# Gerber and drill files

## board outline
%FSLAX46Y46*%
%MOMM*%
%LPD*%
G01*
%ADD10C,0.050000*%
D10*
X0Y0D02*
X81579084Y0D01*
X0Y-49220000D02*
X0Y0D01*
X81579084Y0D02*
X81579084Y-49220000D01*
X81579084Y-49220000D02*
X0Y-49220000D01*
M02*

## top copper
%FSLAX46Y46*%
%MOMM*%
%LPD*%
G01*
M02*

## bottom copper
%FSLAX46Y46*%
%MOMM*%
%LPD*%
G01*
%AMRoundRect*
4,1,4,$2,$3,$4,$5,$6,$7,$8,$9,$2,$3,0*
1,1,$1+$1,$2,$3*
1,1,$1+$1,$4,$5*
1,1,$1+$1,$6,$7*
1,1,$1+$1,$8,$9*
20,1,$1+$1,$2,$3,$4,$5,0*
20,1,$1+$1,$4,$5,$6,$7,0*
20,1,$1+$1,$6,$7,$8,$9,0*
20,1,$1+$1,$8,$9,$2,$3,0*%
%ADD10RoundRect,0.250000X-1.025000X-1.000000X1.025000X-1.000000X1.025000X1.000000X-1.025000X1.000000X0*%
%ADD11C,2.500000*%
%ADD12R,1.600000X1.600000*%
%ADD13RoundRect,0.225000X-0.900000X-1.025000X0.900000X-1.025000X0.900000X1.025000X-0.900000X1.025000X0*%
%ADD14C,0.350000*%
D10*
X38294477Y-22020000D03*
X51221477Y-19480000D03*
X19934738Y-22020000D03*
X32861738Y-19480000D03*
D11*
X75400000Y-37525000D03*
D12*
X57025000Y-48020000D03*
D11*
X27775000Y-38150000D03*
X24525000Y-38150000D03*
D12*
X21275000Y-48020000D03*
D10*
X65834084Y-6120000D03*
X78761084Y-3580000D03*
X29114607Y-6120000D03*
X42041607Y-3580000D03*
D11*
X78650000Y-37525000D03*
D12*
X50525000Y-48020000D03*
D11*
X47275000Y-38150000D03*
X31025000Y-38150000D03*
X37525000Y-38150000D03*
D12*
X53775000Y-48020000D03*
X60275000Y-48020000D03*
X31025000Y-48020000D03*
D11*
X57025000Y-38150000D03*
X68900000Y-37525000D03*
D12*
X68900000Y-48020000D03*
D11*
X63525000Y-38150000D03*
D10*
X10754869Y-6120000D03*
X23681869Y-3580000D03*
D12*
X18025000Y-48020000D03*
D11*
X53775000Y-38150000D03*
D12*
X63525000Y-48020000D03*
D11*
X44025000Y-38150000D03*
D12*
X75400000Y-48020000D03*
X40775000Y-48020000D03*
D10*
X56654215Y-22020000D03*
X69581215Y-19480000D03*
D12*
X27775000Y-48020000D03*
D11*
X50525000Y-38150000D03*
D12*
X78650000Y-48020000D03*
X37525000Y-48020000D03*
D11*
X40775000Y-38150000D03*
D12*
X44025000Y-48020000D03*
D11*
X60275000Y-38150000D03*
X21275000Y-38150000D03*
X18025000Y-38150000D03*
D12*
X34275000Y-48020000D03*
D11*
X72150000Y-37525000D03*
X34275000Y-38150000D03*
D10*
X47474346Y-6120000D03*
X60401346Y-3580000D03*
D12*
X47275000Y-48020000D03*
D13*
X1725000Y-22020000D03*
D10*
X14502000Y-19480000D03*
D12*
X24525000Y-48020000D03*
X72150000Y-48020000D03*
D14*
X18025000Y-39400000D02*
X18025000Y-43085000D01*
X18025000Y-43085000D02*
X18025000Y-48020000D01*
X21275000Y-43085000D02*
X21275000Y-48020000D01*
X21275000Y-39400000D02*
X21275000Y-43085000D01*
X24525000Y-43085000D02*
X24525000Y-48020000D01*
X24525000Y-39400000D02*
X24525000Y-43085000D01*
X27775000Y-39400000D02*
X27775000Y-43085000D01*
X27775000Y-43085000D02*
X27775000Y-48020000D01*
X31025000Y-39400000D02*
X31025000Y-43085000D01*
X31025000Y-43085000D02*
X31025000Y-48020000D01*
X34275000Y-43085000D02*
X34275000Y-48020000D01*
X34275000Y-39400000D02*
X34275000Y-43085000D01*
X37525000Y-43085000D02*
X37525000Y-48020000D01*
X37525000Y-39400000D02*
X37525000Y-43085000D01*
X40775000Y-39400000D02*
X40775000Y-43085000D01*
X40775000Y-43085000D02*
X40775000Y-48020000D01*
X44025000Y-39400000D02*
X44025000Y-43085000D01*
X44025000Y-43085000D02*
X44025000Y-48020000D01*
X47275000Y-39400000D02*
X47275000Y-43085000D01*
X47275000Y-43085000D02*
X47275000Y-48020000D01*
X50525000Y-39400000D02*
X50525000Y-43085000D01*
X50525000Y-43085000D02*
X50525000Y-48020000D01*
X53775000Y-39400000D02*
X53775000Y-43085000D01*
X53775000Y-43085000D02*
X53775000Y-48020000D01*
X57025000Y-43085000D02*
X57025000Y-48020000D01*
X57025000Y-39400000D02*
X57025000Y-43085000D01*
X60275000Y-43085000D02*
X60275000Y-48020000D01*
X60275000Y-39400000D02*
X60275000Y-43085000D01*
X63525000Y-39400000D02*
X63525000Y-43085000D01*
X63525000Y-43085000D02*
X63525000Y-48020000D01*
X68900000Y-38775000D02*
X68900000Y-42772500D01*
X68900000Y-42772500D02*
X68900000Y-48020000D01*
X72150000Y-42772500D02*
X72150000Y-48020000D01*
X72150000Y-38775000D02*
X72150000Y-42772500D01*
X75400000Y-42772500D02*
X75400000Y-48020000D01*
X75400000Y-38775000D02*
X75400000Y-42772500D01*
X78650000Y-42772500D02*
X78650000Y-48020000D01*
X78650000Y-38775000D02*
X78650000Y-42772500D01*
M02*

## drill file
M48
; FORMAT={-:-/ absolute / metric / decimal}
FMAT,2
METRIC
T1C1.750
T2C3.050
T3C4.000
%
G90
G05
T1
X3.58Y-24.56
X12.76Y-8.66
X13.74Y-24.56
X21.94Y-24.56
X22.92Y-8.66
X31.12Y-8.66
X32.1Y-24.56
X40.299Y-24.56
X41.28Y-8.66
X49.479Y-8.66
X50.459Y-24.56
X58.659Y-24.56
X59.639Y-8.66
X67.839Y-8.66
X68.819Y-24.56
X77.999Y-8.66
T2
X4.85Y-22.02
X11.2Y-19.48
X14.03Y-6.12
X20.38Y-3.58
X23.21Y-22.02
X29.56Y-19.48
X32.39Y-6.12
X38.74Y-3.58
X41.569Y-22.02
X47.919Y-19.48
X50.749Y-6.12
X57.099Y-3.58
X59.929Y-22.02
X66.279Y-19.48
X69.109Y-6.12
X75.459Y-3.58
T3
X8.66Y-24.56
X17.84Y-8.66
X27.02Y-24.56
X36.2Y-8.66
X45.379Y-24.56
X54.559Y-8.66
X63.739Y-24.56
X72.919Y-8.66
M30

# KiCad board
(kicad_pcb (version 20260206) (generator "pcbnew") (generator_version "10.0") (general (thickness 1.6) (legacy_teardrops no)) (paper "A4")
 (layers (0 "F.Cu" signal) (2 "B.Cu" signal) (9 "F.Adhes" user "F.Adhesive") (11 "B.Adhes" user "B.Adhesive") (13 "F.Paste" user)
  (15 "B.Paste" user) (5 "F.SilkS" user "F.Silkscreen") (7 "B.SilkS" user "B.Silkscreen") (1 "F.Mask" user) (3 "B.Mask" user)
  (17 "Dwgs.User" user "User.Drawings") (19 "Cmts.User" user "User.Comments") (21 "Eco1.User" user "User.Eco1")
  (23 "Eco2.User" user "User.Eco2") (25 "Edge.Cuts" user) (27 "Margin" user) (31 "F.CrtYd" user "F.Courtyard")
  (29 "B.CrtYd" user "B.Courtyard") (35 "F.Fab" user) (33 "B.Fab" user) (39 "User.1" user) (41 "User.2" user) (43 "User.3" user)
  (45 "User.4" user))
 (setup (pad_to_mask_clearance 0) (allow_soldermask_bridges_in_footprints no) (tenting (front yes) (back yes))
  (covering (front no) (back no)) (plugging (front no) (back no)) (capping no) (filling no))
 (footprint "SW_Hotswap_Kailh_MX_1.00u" (layer "F.Cu") (at 45.379477 24.56)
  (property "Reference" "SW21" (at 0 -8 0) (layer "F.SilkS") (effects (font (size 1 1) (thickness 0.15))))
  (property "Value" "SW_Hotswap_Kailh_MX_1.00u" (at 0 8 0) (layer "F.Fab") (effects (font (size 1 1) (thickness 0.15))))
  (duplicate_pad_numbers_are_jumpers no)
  (pad "" np_thru_hole circle (at -5.08 0) (size 1.75 1.75) (drill 1.75) (layers "*.Cu" "*.Mask"))
  (pad "" np_thru_hole circle (at -3.81 -2.54) (size 3.05 3.05) (drill 3.05) (layers "*.Cu" "*.Mask"))
  (pad "" np_thru_hole circle (at 0 0) (size 4 4) (drill 4) (layers "*.Cu" "*.Mask"))
  (pad "" np_thru_hole circle (at 2.54 -5.08) (size 3.05 3.05) (drill 3.05) (layers "*.Cu" "*.Mask"))
  (pad "" np_thru_hole circle (at 5.08 0) (size 1.75 1.75) (drill 1.75) (layers "*.Cu" "*.Mask"))
  (pad "1" smd roundrect (at -7.085 -2.54) (size 2.55 2.5) (layers "B.Cu" "B.Mask" "B.Paste") (roundrect_rratio 0.1))
  (pad "2" smd roundrect (at 5.842 -5.08) (size 2.55 2.5) (layers "B.Cu" "B.Mask" "B.Paste") (roundrect_rratio 0.1)))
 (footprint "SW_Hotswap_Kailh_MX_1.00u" (layer "F.Cu") (at 27.019738 24.56)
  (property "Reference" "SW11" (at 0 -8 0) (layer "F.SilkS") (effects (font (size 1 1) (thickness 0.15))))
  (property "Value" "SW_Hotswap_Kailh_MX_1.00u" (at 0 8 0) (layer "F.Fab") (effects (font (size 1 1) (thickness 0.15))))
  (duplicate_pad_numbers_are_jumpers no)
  (pad "" np_thru_hole circle (at -5.08 0) (size 1.75 1.75) (drill 1.75) (layers "*.Cu" "*.Mask"))
  (pad "" np_thru_hole circle (at -3.81 -2.54) (size 3.05 3.05) (drill 3.05) (layers "*.Cu" "*.Mask"))
  (pad "" np_thru_hole circle (at 0 0) (size 4 4) (drill 4) (layers "*.Cu" "*.Mask"))
  (pad "" np_thru_hole circle (at 2.54 -5.08) (size 3.05 3.05) (drill 3.05) (layers "*.Cu" "*.Mask"))
  (pad "" np_thru_hole circle (at 5.08 0) (size 1.75 1.75) (drill 1.75) (layers "*.Cu" "*.Mask"))
  (pad "1" smd roundrect (at -7.085 -2.54) (size 2.55 2.5) (layers "B.Cu" "B.Mask" "B.Paste") (roundrect_rratio 0.1))
  (pad "2" smd roundrect (at 5.842 -5.08) (size 2.55 2.5) (layers "B.Cu" "B.Mask" "B.Paste") (roundrect_rratio 0.1)))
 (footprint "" (layer "F.Cu") (at 0 0)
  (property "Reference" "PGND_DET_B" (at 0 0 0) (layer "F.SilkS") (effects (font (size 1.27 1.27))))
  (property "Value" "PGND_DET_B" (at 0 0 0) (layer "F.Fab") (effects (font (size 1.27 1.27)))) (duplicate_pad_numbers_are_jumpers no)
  (pad "1" smd circle (at 75.4 37.525) (size 2.5 2.5) (layers "B.Cu" "B.Mask") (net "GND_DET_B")))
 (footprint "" (layer "F.Cu") (at 0 0)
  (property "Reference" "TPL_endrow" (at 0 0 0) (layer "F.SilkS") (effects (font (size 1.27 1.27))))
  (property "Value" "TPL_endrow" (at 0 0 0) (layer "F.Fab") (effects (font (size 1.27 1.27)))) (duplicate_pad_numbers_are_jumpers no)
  (pad "1" smd rect (at 57.025 48.02) (size 1.6 1.6) (layers "B.Cu" "B.Mask") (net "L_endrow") (thermal_bridge_angle 45)))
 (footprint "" (layer "F.Cu") (at 0 0)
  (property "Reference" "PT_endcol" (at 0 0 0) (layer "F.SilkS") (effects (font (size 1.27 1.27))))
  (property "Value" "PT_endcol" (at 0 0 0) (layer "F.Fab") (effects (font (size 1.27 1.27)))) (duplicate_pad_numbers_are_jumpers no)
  (pad "1" smd circle (at 27.775 38.15) (size 2.5 2.5) (layers "B.Cu" "B.Mask") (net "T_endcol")))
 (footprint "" (layer "F.Cu") (at 0 0)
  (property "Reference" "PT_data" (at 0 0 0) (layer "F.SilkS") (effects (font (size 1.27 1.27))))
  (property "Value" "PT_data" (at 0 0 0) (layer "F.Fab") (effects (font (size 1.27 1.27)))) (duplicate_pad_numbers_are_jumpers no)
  (pad "1" smd circle (at 24.525 38.15) (size 2.5 2.5) (layers "B.Cu" "B.Mask") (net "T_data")))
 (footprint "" (layer "F.Cu") (at 0 0)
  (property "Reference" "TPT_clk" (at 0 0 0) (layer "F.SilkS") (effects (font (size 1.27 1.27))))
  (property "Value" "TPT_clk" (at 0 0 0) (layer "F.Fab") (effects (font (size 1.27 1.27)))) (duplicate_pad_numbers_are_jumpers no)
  (pad "1" smd rect (at 21.275 48.02) (size 1.6 1.6) (layers "B.Cu" "B.Mask") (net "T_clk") (thermal_bridge_angle 45)))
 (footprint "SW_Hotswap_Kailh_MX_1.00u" (layer "F.Cu") (at 72.919084 8.66)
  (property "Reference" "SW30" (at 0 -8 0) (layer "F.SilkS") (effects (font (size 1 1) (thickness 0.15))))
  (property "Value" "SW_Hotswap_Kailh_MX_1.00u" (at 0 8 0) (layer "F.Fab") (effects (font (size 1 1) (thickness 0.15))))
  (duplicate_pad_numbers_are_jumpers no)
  (pad "" np_thru_hole circle (at -5.08 0) (size 1.75 1.75) (drill 1.75) (layers "*.Cu" "*.Mask"))
  (pad "" np_thru_hole circle (at -3.81 -2.54) (size 3.05 3.05) (drill 3.05) (layers "*.Cu" "*.Mask"))
  (pad "" np_thru_hole circle (at 0 0) (size 4 4) (drill 4) (layers "*.Cu" "*.Mask"))
  (pad "" np_thru_hole circle (at 2.54 -5.08) (size 3.05 3.05) (drill 3.05) (layers "*.Cu" "*.Mask"))
  (pad "" np_thru_hole circle (at 5.08 0) (size 1.75 1.75) (drill 1.75) (layers "*.Cu" "*.Mask"))
  (pad "1" smd roundrect (at -7.085 -2.54) (size 2.55 2.5) (layers "B.Cu" "B.Mask" "B.Paste") (roundrect_rratio 0.1))
  (pad "2" smd roundrect (at 5.842 -5.08) (size 2.55 2.5) (layers "B.Cu" "B.Mask" "B.Paste") (roundrect_rratio 0.1)))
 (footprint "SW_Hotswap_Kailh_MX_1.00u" (layer "F.Cu") (at 36.199607 8.66)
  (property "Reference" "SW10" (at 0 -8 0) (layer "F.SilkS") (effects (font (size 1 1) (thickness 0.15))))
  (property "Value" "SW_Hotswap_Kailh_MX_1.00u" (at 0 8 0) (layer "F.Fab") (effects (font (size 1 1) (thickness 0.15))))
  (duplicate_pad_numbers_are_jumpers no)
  (pad "" np_thru_hole circle (at -5.08 0) (size 1.75 1.75) (drill 1.75) (layers "*.Cu" "*.Mask"))
  (pad "" np_thru_hole circle (at -3.81 -2.54) (size 3.05 3.05) (drill 3.05) (layers "*.Cu" "*.Mask"))
  (pad "" np_thru_hole circle (at 0 0) (size 4 4) (drill 4) (layers "*.Cu" "*.Mask"))
  (pad "" np_thru_hole circle (at 2.54 -5.08) (size 3.05 3.05) (drill 3.05) (layers "*.Cu" "*.Mask"))
  (pad "" np_thru_hole circle (at 5.08 0) (size 1.75 1.75) (drill 1.75) (layers "*.Cu" "*.Mask"))
  (pad "1" smd roundrect (at -7.085 -2.54) (size 2.55 2.5) (layers "B.Cu" "B.Mask" "B.Paste") (roundrect_rratio 0.1))
  (pad "2" smd roundrect (at 5.842 -5.08) (size 2.55 2.5) (layers "B.Cu" "B.Mask" "B.Paste") (roundrect_rratio 0.1)))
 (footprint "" (layer "F.Cu") (at 0 0)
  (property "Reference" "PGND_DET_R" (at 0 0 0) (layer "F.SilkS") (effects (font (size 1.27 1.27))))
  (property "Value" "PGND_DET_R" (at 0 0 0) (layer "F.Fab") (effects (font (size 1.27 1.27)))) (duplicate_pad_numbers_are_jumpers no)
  (pad "1" smd circle (at 78.65 37.525) (size 2.5 2.5) (layers "B.Cu" "B.Mask") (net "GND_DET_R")))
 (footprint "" (layer "F.Cu") (at 0 0)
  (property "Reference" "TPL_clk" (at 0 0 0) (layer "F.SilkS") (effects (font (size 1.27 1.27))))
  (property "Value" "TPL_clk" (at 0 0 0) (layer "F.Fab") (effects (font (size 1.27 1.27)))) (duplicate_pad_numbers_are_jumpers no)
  (pad "1" smd rect (at 50.525 48.02) (size 1.6 1.6) (layers "B.Cu" "B.Mask") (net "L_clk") (thermal_bridge_angle 45)))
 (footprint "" (layer "F.Cu") (at 0 0)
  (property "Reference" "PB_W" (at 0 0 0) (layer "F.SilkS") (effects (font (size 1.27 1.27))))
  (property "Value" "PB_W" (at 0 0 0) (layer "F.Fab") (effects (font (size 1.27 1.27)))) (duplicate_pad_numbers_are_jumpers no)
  (pad "1" smd circle (at 47.275 38.15) (size 2.5 2.5) (layers "B.Cu" "B.Mask") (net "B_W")))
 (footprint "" (layer "F.Cu") (at 0 0)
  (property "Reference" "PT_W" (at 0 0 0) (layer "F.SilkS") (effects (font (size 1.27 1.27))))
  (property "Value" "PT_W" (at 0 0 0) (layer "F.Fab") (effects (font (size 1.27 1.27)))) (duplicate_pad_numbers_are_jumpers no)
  (pad "1" smd circle (at 31.025 38.15) (size 2.5 2.5) (layers "B.Cu" "B.Mask") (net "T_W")))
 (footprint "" (layer "F.Cu") (at 0 0)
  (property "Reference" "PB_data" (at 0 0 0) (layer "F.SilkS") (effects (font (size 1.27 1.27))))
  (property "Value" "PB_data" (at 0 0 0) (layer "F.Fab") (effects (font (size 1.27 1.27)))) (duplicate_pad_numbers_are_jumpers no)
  (pad "1" smd circle (at 37.525 38.15) (size 2.5 2.5) (layers "B.Cu" "B.Mask") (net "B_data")))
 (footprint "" (layer "F.Cu") (at 0 0)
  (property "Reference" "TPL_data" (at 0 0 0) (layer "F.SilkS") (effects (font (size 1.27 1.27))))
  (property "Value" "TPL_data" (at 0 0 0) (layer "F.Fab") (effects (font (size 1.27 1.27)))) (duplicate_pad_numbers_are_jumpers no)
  (pad "1" smd rect (at 53.775 48.02) (size 1.6 1.6) (layers "B.Cu" "B.Mask") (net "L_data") (thermal_bridge_angle 45)))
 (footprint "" (layer "F.Cu") (at 0 0)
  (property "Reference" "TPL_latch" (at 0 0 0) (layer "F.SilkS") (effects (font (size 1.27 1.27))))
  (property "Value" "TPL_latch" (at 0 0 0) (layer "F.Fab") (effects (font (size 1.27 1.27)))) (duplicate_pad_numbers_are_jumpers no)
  (pad "1" smd rect (at 60.275 48.02) (size 1.6 1.6) (layers "B.Cu" "B.Mask") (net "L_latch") (thermal_bridge_angle 45)))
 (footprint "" (layer "F.Cu") (at 0 0)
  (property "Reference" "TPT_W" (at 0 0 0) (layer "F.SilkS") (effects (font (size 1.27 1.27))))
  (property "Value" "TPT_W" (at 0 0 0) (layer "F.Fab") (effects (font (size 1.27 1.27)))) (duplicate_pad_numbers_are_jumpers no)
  (pad "1" smd rect (at 31.025 48.02) (size 1.6 1.6) (layers "B.Cu" "B.Mask") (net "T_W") (thermal_bridge_angle 45)))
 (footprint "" (layer "F.Cu") (at 0 0)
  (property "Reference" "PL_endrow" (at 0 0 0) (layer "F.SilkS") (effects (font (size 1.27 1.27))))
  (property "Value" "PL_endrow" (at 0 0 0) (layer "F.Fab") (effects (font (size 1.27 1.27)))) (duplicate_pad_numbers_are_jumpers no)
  (pad "1" smd circle (at 57.025 38.15) (size 2.5 2.5) (layers "B.Cu" "B.Mask") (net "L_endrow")))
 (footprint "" (layer "F.Cu") (at 0 0)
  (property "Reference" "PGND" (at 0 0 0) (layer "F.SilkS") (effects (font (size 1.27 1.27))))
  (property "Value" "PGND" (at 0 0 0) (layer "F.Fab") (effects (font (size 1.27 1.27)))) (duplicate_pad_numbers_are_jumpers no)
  (pad "1" smd circle (at 68.9 37.525) (size 2.5 2.5) (layers "B.Cu" "B.Mask") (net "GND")))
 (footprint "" (layer "F.Cu") (at 0 0)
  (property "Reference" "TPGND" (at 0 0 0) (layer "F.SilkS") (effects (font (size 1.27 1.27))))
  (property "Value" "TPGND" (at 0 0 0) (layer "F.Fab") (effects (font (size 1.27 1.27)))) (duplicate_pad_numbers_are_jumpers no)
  (pad "1" smd rect (at 68.9 48.02) (size 1.6 1.6) (layers "B.Cu" "B.Mask") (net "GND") (thermal_bridge_angle 45)))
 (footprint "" (layer "F.Cu") (at 0 0)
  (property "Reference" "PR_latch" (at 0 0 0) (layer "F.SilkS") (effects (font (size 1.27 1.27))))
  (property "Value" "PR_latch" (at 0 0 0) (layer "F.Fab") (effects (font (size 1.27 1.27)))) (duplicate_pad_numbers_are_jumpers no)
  (pad "1" smd circle (at 63.525 38.15) (size 2.5 2.5) (layers "B.Cu" "B.Mask") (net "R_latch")))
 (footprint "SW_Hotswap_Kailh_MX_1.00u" (layer "F.Cu") (at 17.839869 8.66)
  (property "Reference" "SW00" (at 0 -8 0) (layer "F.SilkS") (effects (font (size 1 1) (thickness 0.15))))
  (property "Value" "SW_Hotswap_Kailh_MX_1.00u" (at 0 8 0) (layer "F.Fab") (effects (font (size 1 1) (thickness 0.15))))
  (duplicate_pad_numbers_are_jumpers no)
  (pad "" np_thru_hole circle (at -5.08 0) (size 1.75 1.75) (drill 1.75) (layers "*.Cu" "*.Mask"))
  (pad "" np_thru_hole circle (at -3.81 -2.54) (size 3.05 3.05) (drill 3.05) (layers "*.Cu" "*.Mask"))
  (pad "" np_thru_hole circle (at 0 0) (size 4 4) (drill 4) (layers "*.Cu" "*.Mask"))
  (pad "" np_thru_hole circle (at 2.54 -5.08) (size 3.05 3.05) (drill 3.05) (layers "*.Cu" "*.Mask"))
  (pad "" np_thru_hole circle (at 5.08 0) (size 1.75 1.75) (drill 1.75) (layers "*.Cu" "*.Mask"))
  (pad "1" smd roundrect (at -7.085 -2.54) (size 2.55 2.5) (layers "B.Cu" "B.Mask" "B.Paste") (roundrect_rratio 0.1))
  (pad "2" smd roundrect (at 5.842 -5.08) (size 2.55 2.5) (layers "B.Cu" "B.Mask" "B.Paste") (roundrect_rratio 0.1)))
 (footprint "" (layer "F.Cu") (at 0 0)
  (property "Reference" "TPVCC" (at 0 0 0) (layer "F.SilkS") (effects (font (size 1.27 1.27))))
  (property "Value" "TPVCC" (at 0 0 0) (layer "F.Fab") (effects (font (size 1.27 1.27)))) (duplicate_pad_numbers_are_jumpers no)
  (pad "1" smd rect (at 18.025 48.02) (size 1.6 1.6) (layers "B.Cu" "B.Mask") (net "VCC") (thermal_bridge_angle 45)))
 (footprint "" (layer "F.Cu") (at 0 0)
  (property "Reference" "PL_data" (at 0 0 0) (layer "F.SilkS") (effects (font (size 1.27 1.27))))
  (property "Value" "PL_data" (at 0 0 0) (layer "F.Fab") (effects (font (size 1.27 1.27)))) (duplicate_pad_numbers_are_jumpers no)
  (pad "1" smd circle (at 53.775 38.15) (size 2.5 2.5) (layers "B.Cu" "B.Mask") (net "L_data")))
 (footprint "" (layer "F.Cu") (at 0 0)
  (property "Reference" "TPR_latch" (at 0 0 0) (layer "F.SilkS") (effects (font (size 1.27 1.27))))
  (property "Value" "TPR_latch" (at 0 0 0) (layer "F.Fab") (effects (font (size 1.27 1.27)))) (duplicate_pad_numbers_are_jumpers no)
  (pad "1" smd rect (at 63.525 48.02) (size 1.6 1.6) (layers "B.Cu" "B.Mask") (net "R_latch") (thermal_bridge_angle 45)))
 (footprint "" (layer "F.Cu") (at 0 0)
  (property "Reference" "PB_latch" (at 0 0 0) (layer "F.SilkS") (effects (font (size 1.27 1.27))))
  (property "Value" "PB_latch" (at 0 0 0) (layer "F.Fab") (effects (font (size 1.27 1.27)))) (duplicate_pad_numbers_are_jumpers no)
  (pad "1" smd circle (at 44.025 38.15) (size 2.5 2.5) (layers "B.Cu" "B.Mask") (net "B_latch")))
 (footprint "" (layer "F.Cu") (at 0 0)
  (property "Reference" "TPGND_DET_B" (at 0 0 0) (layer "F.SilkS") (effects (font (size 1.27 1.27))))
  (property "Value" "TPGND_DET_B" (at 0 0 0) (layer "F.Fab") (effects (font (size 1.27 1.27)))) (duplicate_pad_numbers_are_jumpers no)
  (pad "1" smd rect (at 75.4 48.02) (size 1.6 1.6) (layers "B.Cu" "B.Mask") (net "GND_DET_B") (thermal_bridge_angle 45)))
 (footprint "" (layer "F.Cu") (at 0 0)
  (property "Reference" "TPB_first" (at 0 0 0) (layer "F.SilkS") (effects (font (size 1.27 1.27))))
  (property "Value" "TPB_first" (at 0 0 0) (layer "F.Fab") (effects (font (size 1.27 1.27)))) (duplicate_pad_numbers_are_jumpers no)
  (pad "1" smd rect (at 40.775 48.02) (size 1.6 1.6) (layers "B.Cu" "B.Mask") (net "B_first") (thermal_bridge_angle 45)))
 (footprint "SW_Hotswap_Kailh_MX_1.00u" (layer "F.Cu") (at 63.739215 24.56)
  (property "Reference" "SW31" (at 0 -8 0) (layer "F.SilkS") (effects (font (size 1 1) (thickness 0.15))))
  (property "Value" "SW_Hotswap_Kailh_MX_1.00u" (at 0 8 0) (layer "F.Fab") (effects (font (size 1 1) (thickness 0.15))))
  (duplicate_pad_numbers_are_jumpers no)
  (pad "" np_thru_hole circle (at -5.08 0) (size 1.75 1.75) (drill 1.75) (layers "*.Cu" "*.Mask"))
  (pad "" np_thru_hole circle (at -3.81 -2.54) (size 3.05 3.05) (drill 3.05) (layers "*.Cu" "*.Mask"))
  (pad "" np_thru_hole circle (at 0 0) (size 4 4) (drill 4) (layers "*.Cu" "*.Mask"))
  (pad "" np_thru_hole circle (at 2.54 -5.08) (size 3.05 3.05) (drill 3.05) (layers "*.Cu" "*.Mask"))
  (pad "" np_thru_hole circle (at 5.08 0) (size 1.75 1.75) (drill 1.75) (layers "*.Cu" "*.Mask"))
  (pad "1" smd roundrect (at -7.085 -2.54) (size 2.55 2.5) (layers "B.Cu" "B.Mask" "B.Paste") (roundrect_rratio 0.1))
  (pad "2" smd roundrect (at 5.842 -5.08) (size 2.55 2.5) (layers "B.Cu" "B.Mask" "B.Paste") (roundrect_rratio 0.1)))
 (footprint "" (layer "F.Cu") (at 0 0)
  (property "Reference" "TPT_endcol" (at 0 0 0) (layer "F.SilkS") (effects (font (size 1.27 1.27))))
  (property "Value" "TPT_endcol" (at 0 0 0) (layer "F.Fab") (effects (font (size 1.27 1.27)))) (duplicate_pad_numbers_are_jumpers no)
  (pad "1" smd rect (at 27.775 48.02) (size 1.6 1.6) (layers "B.Cu" "B.Mask") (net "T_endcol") (thermal_bridge_angle 45)))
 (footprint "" (layer "F.Cu") (at 0 0)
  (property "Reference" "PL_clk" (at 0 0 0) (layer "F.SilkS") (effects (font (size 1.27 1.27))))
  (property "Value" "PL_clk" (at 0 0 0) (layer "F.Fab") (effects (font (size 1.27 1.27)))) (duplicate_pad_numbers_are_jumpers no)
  (pad "1" smd circle (at 50.525 38.15) (size 2.5 2.5) (layers "B.Cu" "B.Mask") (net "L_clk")))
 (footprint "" (layer "F.Cu") (at 0 0)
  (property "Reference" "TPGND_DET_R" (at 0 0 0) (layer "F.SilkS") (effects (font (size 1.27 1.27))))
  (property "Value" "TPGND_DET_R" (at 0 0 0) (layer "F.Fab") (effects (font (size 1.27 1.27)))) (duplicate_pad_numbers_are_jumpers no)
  (pad "1" smd rect (at 78.65 48.02) (size 1.6 1.6) (layers "B.Cu" "B.Mask") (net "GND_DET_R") (thermal_bridge_angle 45)))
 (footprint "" (layer "F.Cu") (at 0 0)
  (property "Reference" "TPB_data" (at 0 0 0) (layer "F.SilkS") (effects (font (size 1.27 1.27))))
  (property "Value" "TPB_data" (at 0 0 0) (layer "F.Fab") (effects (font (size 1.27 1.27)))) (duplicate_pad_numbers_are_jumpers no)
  (pad "1" smd rect (at 37.525 48.02) (size 1.6 1.6) (layers "B.Cu" "B.Mask") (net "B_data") (thermal_bridge_angle 45)))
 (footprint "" (layer "F.Cu") (at 0 0)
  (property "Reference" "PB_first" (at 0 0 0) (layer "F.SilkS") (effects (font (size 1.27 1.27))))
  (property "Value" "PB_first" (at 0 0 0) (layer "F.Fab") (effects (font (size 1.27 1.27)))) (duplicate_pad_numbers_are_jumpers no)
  (pad "1" smd circle (at 40.775 38.15) (size 2.5 2.5) (layers "B.Cu" "B.Mask") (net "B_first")))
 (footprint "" (layer "F.Cu") (at 0 0)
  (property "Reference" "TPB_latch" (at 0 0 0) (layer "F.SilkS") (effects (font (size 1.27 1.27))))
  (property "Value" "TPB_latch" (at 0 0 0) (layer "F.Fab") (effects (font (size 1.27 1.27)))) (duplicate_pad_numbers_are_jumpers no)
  (pad "1" smd rect (at 44.025 48.02) (size 1.6 1.6) (layers "B.Cu" "B.Mask") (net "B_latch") (thermal_bridge_angle 45)))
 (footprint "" (layer "F.Cu") (at 0 0)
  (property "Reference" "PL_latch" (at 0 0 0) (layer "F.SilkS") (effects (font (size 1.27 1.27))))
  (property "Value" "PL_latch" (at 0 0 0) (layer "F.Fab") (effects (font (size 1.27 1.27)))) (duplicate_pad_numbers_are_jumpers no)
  (pad "1" smd circle (at 60.275 38.15) (size 2.5 2.5) (layers "B.Cu" "B.Mask") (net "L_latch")))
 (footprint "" (layer "F.Cu") (at 0 0)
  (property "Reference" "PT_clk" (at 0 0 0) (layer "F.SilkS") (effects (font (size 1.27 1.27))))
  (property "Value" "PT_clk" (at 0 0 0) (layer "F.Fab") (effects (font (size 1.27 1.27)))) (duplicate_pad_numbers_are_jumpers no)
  (pad "1" smd circle (at 21.275 38.15) (size 2.5 2.5) (layers "B.Cu" "B.Mask") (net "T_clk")))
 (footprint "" (layer "F.Cu") (at 0 0)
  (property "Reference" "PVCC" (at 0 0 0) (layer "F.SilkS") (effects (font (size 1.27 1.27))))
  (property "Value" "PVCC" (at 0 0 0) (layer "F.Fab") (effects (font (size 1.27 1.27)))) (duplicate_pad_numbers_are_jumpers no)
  (pad "1" smd circle (at 18.025 38.15) (size 2.5 2.5) (layers "B.Cu" "B.Mask") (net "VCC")))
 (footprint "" (layer "F.Cu") (at 0 0)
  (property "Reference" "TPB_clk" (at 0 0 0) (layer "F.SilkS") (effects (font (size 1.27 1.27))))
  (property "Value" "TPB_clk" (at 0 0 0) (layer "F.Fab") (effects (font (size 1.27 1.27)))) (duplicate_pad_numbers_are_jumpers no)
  (pad "1" smd rect (at 34.275 48.02) (size 1.6 1.6) (layers "B.Cu" "B.Mask") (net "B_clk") (thermal_bridge_angle 45)))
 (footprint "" (layer "F.Cu") (at 0 0)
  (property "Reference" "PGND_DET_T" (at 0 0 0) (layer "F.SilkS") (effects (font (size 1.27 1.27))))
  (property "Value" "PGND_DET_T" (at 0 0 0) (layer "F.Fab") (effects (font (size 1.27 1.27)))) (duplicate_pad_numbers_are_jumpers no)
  (pad "1" smd circle (at 72.15 37.525) (size 2.5 2.5) (layers "B.Cu" "B.Mask") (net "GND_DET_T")))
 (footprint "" (layer "F.Cu") (at 0 0)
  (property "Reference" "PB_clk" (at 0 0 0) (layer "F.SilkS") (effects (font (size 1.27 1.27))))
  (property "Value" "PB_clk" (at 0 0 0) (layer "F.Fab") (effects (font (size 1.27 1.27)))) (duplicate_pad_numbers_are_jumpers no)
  (pad "1" smd circle (at 34.275 38.15) (size 2.5 2.5) (layers "B.Cu" "B.Mask") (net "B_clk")))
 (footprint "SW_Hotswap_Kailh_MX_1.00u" (layer "F.Cu") (at 54.559346 8.66)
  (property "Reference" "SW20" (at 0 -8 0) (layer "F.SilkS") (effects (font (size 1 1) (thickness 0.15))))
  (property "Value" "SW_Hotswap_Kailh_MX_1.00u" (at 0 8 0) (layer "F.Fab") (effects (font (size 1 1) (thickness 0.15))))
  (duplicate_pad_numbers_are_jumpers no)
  (pad "" np_thru_hole circle (at -5.08 0) (size 1.75 1.75) (drill 1.75) (layers "*.Cu" "*.Mask"))
  (pad "" np_thru_hole circle (at -3.81 -2.54) (size 3.05 3.05) (drill 3.05) (layers "*.Cu" "*.Mask"))
  (pad "" np_thru_hole circle (at 0 0) (size 4 4) (drill 4) (layers "*.Cu" "*.Mask"))
  (pad "" np_thru_hole circle (at 2.54 -5.08) (size 3.05 3.05) (drill 3.05) (layers "*.Cu" "*.Mask"))
  (pad "" np_thru_hole circle (at 5.08 0) (size 1.75 1.75) (drill 1.75) (layers "*.Cu" "*.Mask"))
  (pad "1" smd roundrect (at -7.085 -2.54) (size 2.55 2.5) (layers "B.Cu" "B.Mask" "B.Paste") (roundrect_rratio 0.1))
  (pad "2" smd roundrect (at 5.842 -5.08) (size 2.55 2.5) (layers "B.Cu" "B.Mask" "B.Paste") (roundrect_rratio 0.1)))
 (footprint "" (layer "F.Cu") (at 0 0)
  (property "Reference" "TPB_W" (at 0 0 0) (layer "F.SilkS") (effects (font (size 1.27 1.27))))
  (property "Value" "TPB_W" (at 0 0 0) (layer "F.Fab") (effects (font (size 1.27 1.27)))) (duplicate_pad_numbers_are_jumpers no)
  (pad "1" smd rect (at 47.275 48.02) (size 1.6 1.6) (layers "B.Cu" "B.Mask") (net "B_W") (thermal_bridge_angle 45)))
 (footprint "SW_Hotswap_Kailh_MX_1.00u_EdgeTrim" (layer "F.Cu") (at 8.66 24.56)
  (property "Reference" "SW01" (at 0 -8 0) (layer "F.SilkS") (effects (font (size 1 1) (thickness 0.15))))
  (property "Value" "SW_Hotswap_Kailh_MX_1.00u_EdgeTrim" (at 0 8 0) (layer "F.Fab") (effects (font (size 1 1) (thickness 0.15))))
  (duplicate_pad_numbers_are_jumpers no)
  (pad "" np_thru_hole circle (at -5.08 0) (size 1.75 1.75) (drill 1.75) (layers "*.Cu" "*.Mask"))
  (pad "" np_thru_hole circle (at -3.81 -2.54) (size 3.05 3.05) (drill 3.05) (layers "*.Cu" "*.Mask"))
  (pad "" np_thru_hole circle (at 0 0) (size 4 4) (drill 4) (layers "*.Cu" "*.Mask"))
  (pad "" np_thru_hole circle (at 2.54 -5.08) (size 3.05 3.05) (drill 3.05) (layers "*.Cu" "*.Mask"))
  (pad "" np_thru_hole circle (at 5.08 0) (size 1.75 1.75) (drill 1.75) (layers "*.Cu" "*.Mask"))
  (pad "1" smd roundrect (at -6.935 -2.54) (size 2.25 2.5) (layers "B.Cu" "B.Mask" "B.Paste") (roundrect_rratio 0.1))
  (pad "2" smd roundrect (at 5.842 -5.08) (size 2.55 2.5) (layers "B.Cu" "B.Mask" "B.Paste") (roundrect_rratio 0.1)))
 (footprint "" (layer "F.Cu") (at 0 0)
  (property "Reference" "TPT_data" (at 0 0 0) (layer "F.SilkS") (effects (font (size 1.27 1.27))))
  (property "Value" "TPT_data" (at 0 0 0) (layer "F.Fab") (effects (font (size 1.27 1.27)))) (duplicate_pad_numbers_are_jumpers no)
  (pad "1" smd rect (at 24.525 48.02) (size 1.6 1.6) (layers "B.Cu" "B.Mask") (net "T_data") (thermal_bridge_angle 45)))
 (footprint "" (layer "F.Cu") (at 0 0)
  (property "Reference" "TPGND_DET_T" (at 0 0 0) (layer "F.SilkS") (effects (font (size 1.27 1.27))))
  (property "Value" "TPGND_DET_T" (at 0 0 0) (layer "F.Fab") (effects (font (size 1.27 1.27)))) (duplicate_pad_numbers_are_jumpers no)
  (pad "1" smd rect (at 72.15 48.02) (size 1.6 1.6) (layers "B.Cu" "B.Mask") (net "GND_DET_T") (thermal_bridge_angle 45)))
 (gr_line (start 0 0) (end 81.579084 0) (stroke (width 0.05) (type default)) (layer "Edge.Cuts"))
 (gr_line (start 0 49.22) (end 0 0) (stroke (width 0.05) (type default)) (layer "Edge.Cuts"))
 (gr_line (start 81.579084 0) (end 81.579084 49.22) (stroke (width 0.05) (type default)) (layer "Edge.Cuts"))
 (gr_line (start 81.579084 49.22) (end 0 49.22) (stroke (width 0.05) (type default)) (layer "Edge.Cuts"))
 (segment (start 18.025 39.4) (end 18.025 43.085) (width 0.35) (layer "B.Cu") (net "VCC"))
 (segment (start 18.025 43.085) (end 18.025 48.02) (width 0.35) (layer "B.Cu") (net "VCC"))
 (segment (start 21.275 43.085) (end 21.275 48.02) (width 0.35) (layer "B.Cu") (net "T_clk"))
 (segment (start 21.275 39.4) (end 21.275 43.085) (width 0.35) (layer "B.Cu") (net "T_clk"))
 (segment (start 24.525 43.085) (end 24.525 48.02) (width 0.35) (layer "B.Cu") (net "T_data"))
 (segment (start 24.525 39.4) (end 24.525 43.085) (width 0.35) (layer "B.Cu") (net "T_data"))
 (segment (start 27.775 39.4) (end 27.775 43.085) (width 0.35) (layer "B.Cu") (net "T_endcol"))
 (segment (start 27.775 43.085) (end 27.775 48.02) (width 0.35) (layer "B.Cu") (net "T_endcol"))
 (segment (start 31.025 39.4) (end 31.025 43.085) (width 0.35) (layer "B.Cu") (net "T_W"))
 (segment (start 31.025 43.085) (end 31.025 48.02) (width 0.35) (layer "B.Cu") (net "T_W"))
 (segment (start 34.275 43.085) (end 34.275 48.02) (width 0.35) (layer "B.Cu") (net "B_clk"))
 (segment (start 34.275 39.4) (end 34.275 43.085) (width 0.35) (layer "B.Cu") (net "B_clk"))
 (segment (start 37.525 43.085) (end 37.525 48.02) (width 0.35) (layer "B.Cu") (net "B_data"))
 (segment (start 37.525 39.4) (end 37.525 43.085) (width 0.35) (layer "B.Cu") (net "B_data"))
 (segment (start 40.775 39.4) (end 40.775 43.085) (width 0.35) (layer "B.Cu") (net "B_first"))
 (segment (start 40.775 43.085) (end 40.775 48.02) (width 0.35) (layer "B.Cu") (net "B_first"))
 (segment (start 44.025 39.4) (end 44.025 43.085) (width 0.35) (layer "B.Cu") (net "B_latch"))
 (segment (start 44.025 43.085) (end 44.025 48.02) (width 0.35) (layer "B.Cu") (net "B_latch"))
 (segment (start 47.275 39.4) (end 47.275 43.085) (width 0.35) (layer "B.Cu") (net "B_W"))
 (segment (start 47.275 43.085) (end 47.275 48.02) (width 0.35) (layer "B.Cu") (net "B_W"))
 (segment (start 50.525 39.4) (end 50.525 43.085) (width 0.35) (layer "B.Cu") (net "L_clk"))
 (segment (start 50.525 43.085) (end 50.525 48.02) (width 0.35) (layer "B.Cu") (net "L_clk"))
 (segment (start 53.775 39.4) (end 53.775 43.085) (width 0.35) (layer "B.Cu") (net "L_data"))
 (segment (start 53.775 43.085) (end 53.775 48.02) (width 0.35) (layer "B.Cu") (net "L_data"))
 (segment (start 57.025 43.085) (end 57.025 48.02) (width 0.35) (layer "B.Cu") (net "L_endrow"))
 (segment (start 57.025 39.4) (end 57.025 43.085) (width 0.35) (layer "B.Cu") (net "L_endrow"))
 (segment (start 60.275 43.085) (end 60.275 48.02) (width 0.35) (layer "B.Cu") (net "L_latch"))
 (segment (start 60.275 39.4) (end 60.275 43.085) (width 0.35) (layer "B.Cu") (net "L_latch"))
 (segment (start 63.525 39.4) (end 63.525 43.085) (width 0.35) (layer "B.Cu") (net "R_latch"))
 (segment (start 63.525 43.085) (end 63.525 48.02) (width 0.35) (layer "B.Cu") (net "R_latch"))
 (segment (start 68.9 38.775) (end 68.9 42.7725) (width 0.35) (layer "B.Cu") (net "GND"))
 (segment (start 68.9 42.7725) (end 68.9 48.02) (width 0.35) (layer "B.Cu") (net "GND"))
 (segment (start 72.15 42.7725) (end 72.15 48.02) (width 0.35) (layer "B.Cu") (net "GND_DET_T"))
 (segment (start 72.15 38.775) (end 72.15 42.7725) (width 0.35) (layer "B.Cu") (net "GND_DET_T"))
 (segment (start 75.4 42.7725) (end 75.4 48.02) (width 0.35) (layer "B.Cu") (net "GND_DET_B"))
 (segment (start 75.4 38.775) (end 75.4 42.7725) (width 0.35) (layer "B.Cu") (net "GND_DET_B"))
 (segment (start 78.65 42.7725) (end 78.65 48.02) (width 0.35) (layer "B.Cu") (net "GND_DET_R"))
 (segment (start 78.65 38.775) (end 78.65 42.7725) (width 0.35) (layer "B.Cu") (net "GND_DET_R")))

